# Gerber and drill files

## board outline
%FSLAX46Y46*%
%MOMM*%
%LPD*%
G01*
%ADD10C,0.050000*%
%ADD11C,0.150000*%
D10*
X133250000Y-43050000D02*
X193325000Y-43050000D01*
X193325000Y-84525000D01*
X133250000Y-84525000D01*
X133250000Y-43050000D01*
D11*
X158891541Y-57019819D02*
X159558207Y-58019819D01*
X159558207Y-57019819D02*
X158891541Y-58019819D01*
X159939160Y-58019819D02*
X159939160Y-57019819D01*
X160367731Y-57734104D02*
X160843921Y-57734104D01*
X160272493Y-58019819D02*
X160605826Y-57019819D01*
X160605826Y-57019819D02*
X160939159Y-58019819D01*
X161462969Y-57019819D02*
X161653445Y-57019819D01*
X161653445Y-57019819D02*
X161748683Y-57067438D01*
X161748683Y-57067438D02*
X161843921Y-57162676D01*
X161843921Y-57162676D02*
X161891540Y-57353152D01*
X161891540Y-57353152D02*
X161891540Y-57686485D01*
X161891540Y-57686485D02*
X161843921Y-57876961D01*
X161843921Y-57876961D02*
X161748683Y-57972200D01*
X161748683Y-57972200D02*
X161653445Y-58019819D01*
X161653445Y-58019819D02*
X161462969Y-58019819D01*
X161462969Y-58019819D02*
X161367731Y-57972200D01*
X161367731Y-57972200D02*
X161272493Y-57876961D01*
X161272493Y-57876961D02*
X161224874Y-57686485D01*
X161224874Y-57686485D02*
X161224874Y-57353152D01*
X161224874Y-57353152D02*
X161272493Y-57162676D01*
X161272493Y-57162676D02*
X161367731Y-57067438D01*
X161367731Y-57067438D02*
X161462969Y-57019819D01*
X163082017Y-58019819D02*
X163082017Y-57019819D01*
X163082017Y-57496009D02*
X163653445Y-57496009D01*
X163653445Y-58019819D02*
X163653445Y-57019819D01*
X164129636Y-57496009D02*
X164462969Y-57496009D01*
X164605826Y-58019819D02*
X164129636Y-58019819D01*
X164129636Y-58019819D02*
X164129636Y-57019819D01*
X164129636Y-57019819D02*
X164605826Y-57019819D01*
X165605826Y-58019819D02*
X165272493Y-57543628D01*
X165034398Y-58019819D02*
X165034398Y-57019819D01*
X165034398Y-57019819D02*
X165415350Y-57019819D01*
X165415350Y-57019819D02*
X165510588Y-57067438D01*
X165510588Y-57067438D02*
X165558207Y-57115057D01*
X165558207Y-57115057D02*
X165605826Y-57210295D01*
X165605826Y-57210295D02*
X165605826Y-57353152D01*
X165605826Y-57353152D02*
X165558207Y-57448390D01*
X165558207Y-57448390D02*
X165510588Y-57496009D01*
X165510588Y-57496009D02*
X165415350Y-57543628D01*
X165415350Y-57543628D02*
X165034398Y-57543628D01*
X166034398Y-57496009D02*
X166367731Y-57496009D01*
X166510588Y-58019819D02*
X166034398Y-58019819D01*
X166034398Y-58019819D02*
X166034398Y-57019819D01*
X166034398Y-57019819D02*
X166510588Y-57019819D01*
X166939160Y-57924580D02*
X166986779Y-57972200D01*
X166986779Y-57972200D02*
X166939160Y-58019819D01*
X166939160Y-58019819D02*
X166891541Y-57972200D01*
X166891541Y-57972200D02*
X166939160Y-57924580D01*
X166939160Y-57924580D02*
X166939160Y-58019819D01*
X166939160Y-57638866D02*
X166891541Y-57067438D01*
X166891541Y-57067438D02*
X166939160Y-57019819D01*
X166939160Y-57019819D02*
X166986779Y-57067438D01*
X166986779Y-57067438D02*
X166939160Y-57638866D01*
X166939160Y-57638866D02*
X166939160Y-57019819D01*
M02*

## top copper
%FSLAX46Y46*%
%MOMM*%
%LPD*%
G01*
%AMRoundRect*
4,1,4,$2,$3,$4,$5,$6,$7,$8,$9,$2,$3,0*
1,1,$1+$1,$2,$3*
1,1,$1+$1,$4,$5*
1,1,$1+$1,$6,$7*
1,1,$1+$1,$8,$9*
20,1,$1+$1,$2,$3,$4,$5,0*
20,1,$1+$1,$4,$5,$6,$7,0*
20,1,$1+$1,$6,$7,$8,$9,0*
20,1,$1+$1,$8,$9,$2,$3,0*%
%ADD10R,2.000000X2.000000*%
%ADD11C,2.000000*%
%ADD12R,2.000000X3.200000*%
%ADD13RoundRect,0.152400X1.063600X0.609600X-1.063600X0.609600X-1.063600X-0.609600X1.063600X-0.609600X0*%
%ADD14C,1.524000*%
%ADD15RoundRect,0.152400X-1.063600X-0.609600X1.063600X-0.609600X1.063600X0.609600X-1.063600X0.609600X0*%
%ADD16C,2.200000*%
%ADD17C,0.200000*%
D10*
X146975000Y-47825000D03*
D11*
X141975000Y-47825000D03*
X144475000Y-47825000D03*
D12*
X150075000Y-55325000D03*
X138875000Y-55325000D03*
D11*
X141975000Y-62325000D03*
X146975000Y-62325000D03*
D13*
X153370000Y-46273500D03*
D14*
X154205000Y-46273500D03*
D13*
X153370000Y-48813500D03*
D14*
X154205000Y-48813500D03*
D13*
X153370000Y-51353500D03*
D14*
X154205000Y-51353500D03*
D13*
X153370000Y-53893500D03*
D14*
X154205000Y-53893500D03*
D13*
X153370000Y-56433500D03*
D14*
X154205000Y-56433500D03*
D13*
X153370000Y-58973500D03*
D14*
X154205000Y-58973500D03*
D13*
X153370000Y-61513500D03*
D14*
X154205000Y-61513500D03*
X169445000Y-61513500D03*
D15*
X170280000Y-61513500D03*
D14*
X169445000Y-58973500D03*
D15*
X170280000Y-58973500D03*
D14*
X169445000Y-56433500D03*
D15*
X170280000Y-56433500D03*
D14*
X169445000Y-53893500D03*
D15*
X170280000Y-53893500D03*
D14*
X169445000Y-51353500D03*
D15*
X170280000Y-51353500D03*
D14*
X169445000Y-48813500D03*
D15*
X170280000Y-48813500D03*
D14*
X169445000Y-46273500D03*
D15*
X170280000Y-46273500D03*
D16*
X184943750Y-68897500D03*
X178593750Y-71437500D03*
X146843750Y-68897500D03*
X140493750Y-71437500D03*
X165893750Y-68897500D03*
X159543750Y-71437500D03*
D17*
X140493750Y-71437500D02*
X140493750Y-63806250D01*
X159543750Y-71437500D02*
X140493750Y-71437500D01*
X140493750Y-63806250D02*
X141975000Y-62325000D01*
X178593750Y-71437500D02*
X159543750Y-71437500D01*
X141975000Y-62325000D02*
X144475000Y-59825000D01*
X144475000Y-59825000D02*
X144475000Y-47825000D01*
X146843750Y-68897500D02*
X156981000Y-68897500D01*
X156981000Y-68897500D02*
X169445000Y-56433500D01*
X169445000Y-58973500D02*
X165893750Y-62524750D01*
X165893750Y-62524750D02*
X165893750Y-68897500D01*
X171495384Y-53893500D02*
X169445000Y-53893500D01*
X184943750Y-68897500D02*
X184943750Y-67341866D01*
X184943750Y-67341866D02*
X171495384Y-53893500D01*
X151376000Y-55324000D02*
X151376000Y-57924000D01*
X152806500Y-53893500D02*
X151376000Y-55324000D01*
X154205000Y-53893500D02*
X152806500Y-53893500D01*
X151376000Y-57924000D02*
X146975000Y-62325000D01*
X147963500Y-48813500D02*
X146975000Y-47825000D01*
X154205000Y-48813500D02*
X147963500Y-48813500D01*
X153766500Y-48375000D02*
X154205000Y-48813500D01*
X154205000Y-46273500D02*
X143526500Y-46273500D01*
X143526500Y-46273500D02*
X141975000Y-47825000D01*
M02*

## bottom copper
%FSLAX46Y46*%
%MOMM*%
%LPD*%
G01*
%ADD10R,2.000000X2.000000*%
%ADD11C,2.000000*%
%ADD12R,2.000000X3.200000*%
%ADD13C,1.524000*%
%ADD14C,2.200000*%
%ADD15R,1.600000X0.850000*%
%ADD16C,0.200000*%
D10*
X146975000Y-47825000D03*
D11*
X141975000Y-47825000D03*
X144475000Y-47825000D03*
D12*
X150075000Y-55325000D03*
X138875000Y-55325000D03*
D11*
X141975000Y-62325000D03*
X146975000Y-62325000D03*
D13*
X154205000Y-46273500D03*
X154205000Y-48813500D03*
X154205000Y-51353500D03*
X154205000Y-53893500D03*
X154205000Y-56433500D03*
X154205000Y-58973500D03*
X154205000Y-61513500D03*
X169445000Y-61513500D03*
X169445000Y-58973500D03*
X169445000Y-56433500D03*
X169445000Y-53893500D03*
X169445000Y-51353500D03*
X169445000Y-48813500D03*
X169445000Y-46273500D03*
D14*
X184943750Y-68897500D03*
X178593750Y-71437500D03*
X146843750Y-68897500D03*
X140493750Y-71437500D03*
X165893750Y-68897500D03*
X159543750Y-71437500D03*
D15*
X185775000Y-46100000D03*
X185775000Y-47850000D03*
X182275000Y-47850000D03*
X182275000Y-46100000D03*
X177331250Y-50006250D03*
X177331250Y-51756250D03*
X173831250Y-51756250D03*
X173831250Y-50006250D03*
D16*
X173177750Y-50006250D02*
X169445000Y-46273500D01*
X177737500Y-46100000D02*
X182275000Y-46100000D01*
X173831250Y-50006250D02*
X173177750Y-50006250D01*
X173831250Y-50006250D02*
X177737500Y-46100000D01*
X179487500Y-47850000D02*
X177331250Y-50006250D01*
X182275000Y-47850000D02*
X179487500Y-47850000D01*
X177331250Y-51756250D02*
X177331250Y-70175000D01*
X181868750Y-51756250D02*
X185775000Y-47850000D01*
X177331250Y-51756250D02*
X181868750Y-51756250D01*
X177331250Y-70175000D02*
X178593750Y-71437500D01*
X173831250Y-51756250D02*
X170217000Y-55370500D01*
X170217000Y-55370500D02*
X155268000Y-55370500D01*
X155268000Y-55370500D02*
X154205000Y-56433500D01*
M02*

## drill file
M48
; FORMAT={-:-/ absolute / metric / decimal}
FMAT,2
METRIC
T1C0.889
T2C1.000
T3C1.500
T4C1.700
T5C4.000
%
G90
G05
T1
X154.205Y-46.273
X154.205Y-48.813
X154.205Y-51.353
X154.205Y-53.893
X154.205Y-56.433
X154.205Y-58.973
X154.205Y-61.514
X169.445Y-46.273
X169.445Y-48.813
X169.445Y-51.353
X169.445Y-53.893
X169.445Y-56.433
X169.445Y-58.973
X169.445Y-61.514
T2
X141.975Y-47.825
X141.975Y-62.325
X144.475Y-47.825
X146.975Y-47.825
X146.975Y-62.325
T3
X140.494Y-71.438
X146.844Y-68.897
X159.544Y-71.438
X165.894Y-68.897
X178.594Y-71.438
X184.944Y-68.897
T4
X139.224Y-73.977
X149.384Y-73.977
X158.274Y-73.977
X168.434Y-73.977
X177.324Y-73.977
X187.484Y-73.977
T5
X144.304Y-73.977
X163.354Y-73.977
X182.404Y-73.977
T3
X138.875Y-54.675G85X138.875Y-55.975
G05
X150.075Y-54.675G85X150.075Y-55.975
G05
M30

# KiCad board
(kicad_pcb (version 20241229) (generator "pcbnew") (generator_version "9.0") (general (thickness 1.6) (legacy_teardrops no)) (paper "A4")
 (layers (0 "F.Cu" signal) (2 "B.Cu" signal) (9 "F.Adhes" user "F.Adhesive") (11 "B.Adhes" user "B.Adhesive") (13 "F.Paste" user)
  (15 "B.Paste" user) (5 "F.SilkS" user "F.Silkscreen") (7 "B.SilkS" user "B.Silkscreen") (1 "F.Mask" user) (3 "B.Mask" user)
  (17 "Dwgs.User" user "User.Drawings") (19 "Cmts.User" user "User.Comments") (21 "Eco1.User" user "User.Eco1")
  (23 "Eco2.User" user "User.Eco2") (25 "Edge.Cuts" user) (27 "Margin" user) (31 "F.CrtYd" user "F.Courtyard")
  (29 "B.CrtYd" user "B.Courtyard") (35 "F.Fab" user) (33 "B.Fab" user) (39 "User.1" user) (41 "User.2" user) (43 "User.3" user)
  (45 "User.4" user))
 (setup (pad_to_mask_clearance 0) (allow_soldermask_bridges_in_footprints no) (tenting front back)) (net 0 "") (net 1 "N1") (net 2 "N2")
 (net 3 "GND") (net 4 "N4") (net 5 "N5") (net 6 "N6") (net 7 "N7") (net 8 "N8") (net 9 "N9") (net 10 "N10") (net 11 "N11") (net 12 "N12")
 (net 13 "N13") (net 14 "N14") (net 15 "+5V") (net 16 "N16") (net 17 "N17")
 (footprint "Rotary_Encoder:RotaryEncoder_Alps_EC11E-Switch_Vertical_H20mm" (layer "F.Cu") (at 146.975 47.825 -90)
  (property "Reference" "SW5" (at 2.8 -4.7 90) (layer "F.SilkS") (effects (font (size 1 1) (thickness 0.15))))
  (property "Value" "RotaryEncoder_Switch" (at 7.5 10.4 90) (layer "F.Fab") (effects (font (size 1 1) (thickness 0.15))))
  (pad "A" thru_hole rect (at 0 0 270) (size 2 2) (drill 1) (layers "*.Cu" "*.Mask") (remove_unused_layers no) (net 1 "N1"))
  (pad "B" thru_hole circle (at 0 5 270) (size 2 2) (drill 1) (layers "*.Cu" "*.Mask") (remove_unused_layers no) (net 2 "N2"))
  (pad "C" thru_hole circle (at 0 2.5 270) (size 2 2) (drill 1) (layers "*.Cu" "*.Mask") (remove_unused_layers no) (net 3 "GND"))
  (pad "MP" thru_hole rect (at 7.5 -3.1 270) (size 3.2 2) (drill oval 2.8 1.5) (layers "*.Cu" "*.Mask") (remove_unused_layers no))
  (pad "MP" thru_hole rect (at 7.5 8.1 270) (size 3.2 2) (drill oval 2.8 1.5) (layers "*.Cu" "*.Mask") (remove_unused_layers no))
  (pad "S1" thru_hole circle (at 14.5 5 270) (size 2 2) (drill 1) (layers "*.Cu" "*.Mask") (remove_unused_layers no) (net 3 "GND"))
  (pad "S2" thru_hole circle (at 14.5 0 270) (size 2 2) (drill 1) (layers "*.Cu" "*.Mask") (remove_unused_layers no) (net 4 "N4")))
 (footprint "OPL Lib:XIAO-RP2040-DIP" (layer "F.Cu") (at 161.825 53.8935)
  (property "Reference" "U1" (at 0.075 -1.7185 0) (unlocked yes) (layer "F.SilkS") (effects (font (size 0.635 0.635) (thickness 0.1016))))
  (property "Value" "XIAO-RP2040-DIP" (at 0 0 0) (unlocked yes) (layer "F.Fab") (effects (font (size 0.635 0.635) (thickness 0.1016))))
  (pad "1" smd roundrect (at -8.455 -7.62 180) (size 2.432 1.524) (layers "F.Cu" "F.Mask") (roundrect_rratio 0.1) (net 2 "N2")
   (thermal_bridge_angle 45))
  (pad "1" thru_hole circle (at -7.62 -7.62 180) (size 1.524 1.524) (drill 0.889) (layers "*.Cu" "*.Mask") (remove_unused_layers no)
   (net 2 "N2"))
  (pad "2" smd roundrect (at -8.455 -5.08 180) (size 2.432 1.524) (layers "F.Cu" "F.Mask") (roundrect_rratio 0.1) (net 1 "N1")
   (thermal_bridge_angle 45))
  (pad "2" thru_hole circle (at -7.62 -5.08 180) (size 1.524 1.524) (drill 0.889) (layers "*.Cu" "*.Mask") (remove_unused_layers no)
   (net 1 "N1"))
  (pad "3" smd roundrect (at -8.455 -2.54 180) (size 2.432 1.524) (layers "F.Cu" "F.Mask") (roundrect_rratio 0.1) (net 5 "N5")
   (thermal_bridge_angle 45))
  (pad "3" thru_hole circle (at -7.62 -2.54 180) (size 1.524 1.524) (drill 0.889) (layers "*.Cu" "*.Mask") (remove_unused_layers no)
   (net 5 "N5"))
  (pad "4" smd roundrect (at -8.455 0 180) (size 2.432 1.524) (layers "F.Cu" "F.Mask") (roundrect_rratio 0.1) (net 4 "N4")
   (thermal_bridge_angle 45))
  (pad "4" thru_hole circle (at -7.62 0 180) (size 1.524 1.524) (drill 0.889) (layers "*.Cu" "*.Mask") (remove_unused_layers no)
   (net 4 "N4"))
  (pad "5" smd roundrect (at -8.455 2.54 180) (size 2.432 1.524) (layers "F.Cu" "F.Mask") (roundrect_rratio 0.1) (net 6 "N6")
   (thermal_bridge_angle 45))
  (pad "5" thru_hole circle (at -7.62 2.54 180) (size 1.524 1.524) (drill 0.889) (layers "*.Cu" "*.Mask") (remove_unused_layers no)
   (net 6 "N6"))
  (pad "6" smd roundrect (at -8.455 5.08 180) (size 2.432 1.524) (layers "F.Cu" "F.Mask") (roundrect_rratio 0.1) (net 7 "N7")
   (thermal_bridge_angle 45))
  (pad "6" thru_hole circle (at -7.62 5.08 180) (size 1.524 1.524) (drill 0.889) (layers "*.Cu" "*.Mask") (remove_unused_layers no)
   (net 7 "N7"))
  (pad "7" smd roundrect (at -8.455 7.62 180) (size 2.432 1.524) (layers "F.Cu" "F.Mask") (roundrect_rratio 0.1) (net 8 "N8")
   (thermal_bridge_angle 45))
  (pad "7" thru_hole circle (at -7.62 7.62 180) (size 1.524 1.524) (drill 0.889) (layers "*.Cu" "*.Mask") (remove_unused_layers no)
   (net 8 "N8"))
  (pad "8" thru_hole circle (at 7.62 7.62) (size 1.524 1.524) (drill 0.889) (layers "*.Cu" "*.Mask") (remove_unused_layers no) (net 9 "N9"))
  (pad "8" smd roundrect (at 8.455 7.62) (size 2.432 1.524) (layers "F.Cu" "F.Mask") (roundrect_rratio 0.1) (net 9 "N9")
   (thermal_bridge_angle 45))
  (pad "9" thru_hole circle (at 7.62 5.08) (size 1.524 1.524) (drill 0.889) (layers "*.Cu" "*.Mask") (remove_unused_layers no)
   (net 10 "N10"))
  (pad "9" smd roundrect (at 8.455 5.08) (size 2.432 1.524) (layers "F.Cu" "F.Mask") (roundrect_rratio 0.1) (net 10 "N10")
   (thermal_bridge_angle 45))
  (pad "10" thru_hole circle (at 7.62 2.54) (size 1.524 1.524) (drill 0.889) (layers "*.Cu" "*.Mask") (remove_unused_layers no)
   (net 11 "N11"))
  (pad "10" smd roundrect (at 8.455 2.54) (size 2.432 1.524) (layers "F.Cu" "F.Mask") (roundrect_rratio 0.1) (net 11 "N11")
   (thermal_bridge_angle 45))
  (pad "11" thru_hole circle (at 7.62 0) (size 1.524 1.524) (drill 0.889) (layers "*.Cu" "*.Mask") (remove_unused_layers no) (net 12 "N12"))
  (pad "11" smd roundrect (at 8.455 0) (size 2.432 1.524) (layers "F.Cu" "F.Mask") (roundrect_rratio 0.1) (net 12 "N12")
   (thermal_bridge_angle 45))
  (pad "12" thru_hole circle (at 7.62 -2.54) (size 1.524 1.524) (drill 0.889) (layers "*.Cu" "*.Mask") (remove_unused_layers no)
   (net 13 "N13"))
  (pad "12" smd roundrect (at 8.455 -2.54) (size 2.432 1.524) (layers "F.Cu" "F.Mask") (roundrect_rratio 0.1) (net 13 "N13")
   (thermal_bridge_angle 45))
  (pad "13" thru_hole circle (at 7.62 -5.08) (size 1.524 1.524) (drill 0.889) (layers "*.Cu" "*.Mask") (remove_unused_layers no)
   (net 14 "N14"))
  (pad "13" smd roundrect (at 8.455 -5.08) (size 2.432 1.524) (layers "F.Cu" "F.Mask") (roundrect_rratio 0.1) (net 14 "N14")
   (thermal_bridge_angle 45))
  (pad "14" thru_hole circle (at 7.62 -7.62) (size 1.524 1.524) (drill 0.889) (layers "*.Cu" "*.Mask") (remove_unused_layers no)
   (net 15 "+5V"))
  (pad "14" smd roundrect (at 8.455 -7.62) (size 2.432 1.524) (layers "F.Cu" "F.Mask") (roundrect_rratio 0.1) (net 15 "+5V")
   (thermal_bridge_angle 45)))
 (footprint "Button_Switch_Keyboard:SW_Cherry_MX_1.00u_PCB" (layer "F.Cu") (at 184.94375 68.8975)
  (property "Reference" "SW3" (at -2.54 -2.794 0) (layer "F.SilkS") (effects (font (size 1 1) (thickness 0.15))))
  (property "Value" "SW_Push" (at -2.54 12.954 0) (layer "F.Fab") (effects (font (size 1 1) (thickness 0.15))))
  (pad "" np_thru_hole circle (at -7.62 5.08) (size 1.7 1.7) (drill 1.7) (layers "*.Cu" "*.Mask"))
  (pad "" np_thru_hole circle (at -2.54 5.08) (size 4 4) (drill 4) (layers "*.Cu" "*.Mask"))
  (pad "" np_thru_hole circle (at 2.54 5.08) (size 1.7 1.7) (drill 1.7) (layers "*.Cu" "*.Mask"))
  (pad "1" thru_hole circle (at 0 0) (size 2.2 2.2) (drill 1.5) (layers "*.Cu" "*.Mask") (remove_unused_layers no) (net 12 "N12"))
  (pad "2" thru_hole circle (at -6.35 2.54) (size 2.2 2.2) (drill 1.5) (layers "*.Cu" "*.Mask") (remove_unused_layers no) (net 3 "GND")))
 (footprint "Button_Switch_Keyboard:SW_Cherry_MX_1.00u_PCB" (layer "F.Cu") (at 146.84375 68.8975)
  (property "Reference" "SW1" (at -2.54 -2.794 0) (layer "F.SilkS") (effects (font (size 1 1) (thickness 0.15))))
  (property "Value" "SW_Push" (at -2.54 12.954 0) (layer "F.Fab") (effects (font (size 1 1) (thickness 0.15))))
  (pad "" np_thru_hole circle (at -7.62 5.08) (size 1.7 1.7) (drill 1.7) (layers "*.Cu" "*.Mask"))
  (pad "" np_thru_hole circle (at -2.54 5.08) (size 4 4) (drill 4) (layers "*.Cu" "*.Mask"))
  (pad "" np_thru_hole circle (at 2.54 5.08) (size 1.7 1.7) (drill 1.7) (layers "*.Cu" "*.Mask"))
  (pad "1" thru_hole circle (at 0 0) (size 2.2 2.2) (drill 1.5) (layers "*.Cu" "*.Mask") (remove_unused_layers no) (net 11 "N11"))
  (pad "2" thru_hole circle (at -6.35 2.54) (size 2.2 2.2) (drill 1.5) (layers "*.Cu" "*.Mask") (remove_unused_layers no) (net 3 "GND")))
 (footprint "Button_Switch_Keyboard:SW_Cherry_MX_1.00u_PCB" (layer "F.Cu") (at 165.89375 68.8975)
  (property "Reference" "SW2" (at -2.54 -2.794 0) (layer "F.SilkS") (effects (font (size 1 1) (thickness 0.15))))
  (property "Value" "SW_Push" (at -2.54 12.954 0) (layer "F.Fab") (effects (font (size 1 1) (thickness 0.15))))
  (pad "" np_thru_hole circle (at -7.62 5.08) (size 1.7 1.7) (drill 1.7) (layers "*.Cu" "*.Mask"))
  (pad "" np_thru_hole circle (at -2.54 5.08) (size 4 4) (drill 4) (layers "*.Cu" "*.Mask"))
  (pad "" np_thru_hole circle (at 2.54 5.08) (size 1.7 1.7) (drill 1.7) (layers "*.Cu" "*.Mask"))
  (pad "1" thru_hole circle (at 0 0) (size 2.2 2.2) (drill 1.5) (layers "*.Cu" "*.Mask") (remove_unused_layers no) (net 10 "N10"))
  (pad "2" thru_hole circle (at -6.35 2.54) (size 2.2 2.2) (drill 1.5) (layers "*.Cu" "*.Mask") (remove_unused_layers no) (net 3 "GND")))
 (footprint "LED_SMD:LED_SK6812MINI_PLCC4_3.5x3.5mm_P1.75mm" (layer "B.Cu") (at 184.025 46.975 180)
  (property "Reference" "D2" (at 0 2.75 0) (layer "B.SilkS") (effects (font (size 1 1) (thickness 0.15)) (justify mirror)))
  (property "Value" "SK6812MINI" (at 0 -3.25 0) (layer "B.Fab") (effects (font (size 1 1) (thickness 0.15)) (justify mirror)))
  (pad "1" smd rect (at -1.75 0.875 180) (size 1.6 0.85) (layers "B.Cu" "B.Mask" "B.Paste") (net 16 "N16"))
  (pad "2" smd rect (at -1.75 -0.875 180) (size 1.6 0.85) (layers "B.Cu" "B.Mask" "B.Paste") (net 3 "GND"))
  (pad "3" smd rect (at 1.75 -0.875 180) (size 1.6 0.85) (layers "B.Cu" "B.Mask" "B.Paste") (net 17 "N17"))
  (pad "4" smd rect (at 1.75 0.875 180) (size 1.6 0.85) (layers "B.Cu" "B.Mask" "B.Paste") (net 15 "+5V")))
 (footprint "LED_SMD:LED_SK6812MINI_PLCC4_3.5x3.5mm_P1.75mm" (layer "B.Cu") (at 175.58125 50.88125 180)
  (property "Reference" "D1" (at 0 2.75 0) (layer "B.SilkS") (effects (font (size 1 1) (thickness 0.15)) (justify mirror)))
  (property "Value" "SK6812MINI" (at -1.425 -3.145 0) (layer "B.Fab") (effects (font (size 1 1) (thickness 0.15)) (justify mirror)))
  (pad "1" smd rect (at -1.75 0.875 180) (size 1.6 0.85) (layers "B.Cu" "B.Mask" "B.Paste") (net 17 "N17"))
  (pad "2" smd rect (at -1.75 -0.875 180) (size 1.6 0.85) (layers "B.Cu" "B.Mask" "B.Paste") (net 3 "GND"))
  (pad "3" smd rect (at 1.75 -0.875 180) (size 1.6 0.85) (layers "B.Cu" "B.Mask" "B.Paste") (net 6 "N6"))
  (pad "4" smd rect (at 1.75 0.875 180) (size 1.6 0.85) (layers "B.Cu" "B.Mask" "B.Paste") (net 15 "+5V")))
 (gr_rect (start 133.25 43.05) (end 193.325 84.525) (stroke (width 0.05) (type default)) (fill no) (layer "Edge.Cuts"))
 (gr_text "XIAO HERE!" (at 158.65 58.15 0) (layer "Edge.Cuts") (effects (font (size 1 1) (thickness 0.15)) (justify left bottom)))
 (segment (start 173.17775 50.00625) (end 169.445 46.2735) (width 0.2) (layer "B.Cu") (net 15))
 (segment (start 177.7375 46.1) (end 182.275 46.1) (width 0.2) (layer "B.Cu") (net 15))
 (segment (start 173.83125 50.00625) (end 173.17775 50.00625) (width 0.2) (layer "B.Cu") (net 15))
 (segment (start 173.83125 50.00625) (end 177.7375 46.1) (width 0.2) (layer "B.Cu") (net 15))
 (segment (start 179.4875 47.85) (end 177.33125 50.00625) (width 0.2) (layer "B.Cu") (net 17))
 (segment (start 182.275 47.85) (end 179.4875 47.85) (width 0.2) (layer "B.Cu") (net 17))
 (segment (start 140.49375 71.4375) (end 140.49375 63.80625) (width 0.2) (layer "F.Cu") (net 3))
 (segment (start 159.54375 71.4375) (end 140.49375 71.4375) (width 0.2) (layer "F.Cu") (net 3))
 (segment (start 140.49375 63.80625) (end 141.975 62.325) (width 0.2) (layer "F.Cu") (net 3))
 (segment (start 178.59375 71.4375) (end 159.54375 71.4375) (width 0.2) (layer "F.Cu") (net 3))
 (segment (start 141.975 62.325) (end 144.475 59.825) (width 0.2) (layer "F.Cu") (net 3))
 (segment (start 144.475 59.825) (end 144.475 47.825) (width 0.2) (layer "F.Cu") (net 3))
 (segment (start 177.33125 51.75625) (end 177.33125 70.175) (width 0.2) (layer "B.Cu") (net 3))
 (segment (start 181.86875 51.75625) (end 185.775 47.85) (width 0.2) (layer "B.Cu") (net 3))
 (segment (start 177.33125 51.75625) (end 181.86875 51.75625) (width 0.2) (layer "B.Cu") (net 3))
 (segment (start 177.33125 70.175) (end 178.59375 71.4375) (width 0.2) (layer "B.Cu") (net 3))
 (segment (start 173.83125 51.75625) (end 170.217 55.3705) (width 0.2) (layer "B.Cu") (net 6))
 (segment (start 170.217 55.3705) (end 155.268 55.3705) (width 0.2) (layer "B.Cu") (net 6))
 (segment (start 155.268 55.3705) (end 154.205 56.4335) (width 0.2) (layer "B.Cu") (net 6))
 (segment (start 146.84375 68.8975) (end 156.981 68.8975) (width 0.2) (layer "F.Cu") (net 11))
 (segment (start 156.981 68.8975) (end 169.445 56.4335) (width 0.2) (layer "F.Cu") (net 11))
 (segment (start 169.445 58.9735) (end 165.89375 62.52475) (width 0.2) (layer "F.Cu") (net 10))
 (segment (start 165.89375 62.52475) (end 165.89375 68.8975) (width 0.2) (layer "F.Cu") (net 10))
 (segment (start 171.495384 53.8935) (end 169.445 53.8935) (width 0.2) (layer "F.Cu") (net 12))
 (segment (start 184.94375 68.8975) (end 184.94375 67.341866) (width 0.2) (layer "F.Cu") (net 12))
 (segment (start 184.94375 67.341866) (end 171.495384 53.8935) (width 0.2) (layer "F.Cu") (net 12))
 (segment (start 151.376 55.324) (end 151.376 57.924) (width 0.2) (layer "F.Cu") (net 4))
 (segment (start 152.8065 53.8935) (end 151.376 55.324) (width 0.2) (layer "F.Cu") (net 4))
 (segment (start 154.205 53.8935) (end 152.8065 53.8935) (width 0.2) (layer "F.Cu") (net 4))
 (segment (start 151.376 57.924) (end 146.975 62.325) (width 0.2) (layer "F.Cu") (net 4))
 (segment (start 147.9635 48.8135) (end 146.975 47.825) (width 0.2) (layer "F.Cu") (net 1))
 (segment (start 154.205 48.8135) (end 147.9635 48.8135) (width 0.2) (layer "F.Cu") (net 1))
 (segment (start 153.7665 48.375) (end 154.205 48.8135) (width 0.2) (layer "F.Cu") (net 1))
 (segment (start 154.205 46.2735) (end 143.5265 46.2735) (width 0.2) (layer "F.Cu") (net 2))
 (segment (start 143.5265 46.2735) (end 141.975 47.825) (width 0.2) (layer "F.Cu") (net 2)))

